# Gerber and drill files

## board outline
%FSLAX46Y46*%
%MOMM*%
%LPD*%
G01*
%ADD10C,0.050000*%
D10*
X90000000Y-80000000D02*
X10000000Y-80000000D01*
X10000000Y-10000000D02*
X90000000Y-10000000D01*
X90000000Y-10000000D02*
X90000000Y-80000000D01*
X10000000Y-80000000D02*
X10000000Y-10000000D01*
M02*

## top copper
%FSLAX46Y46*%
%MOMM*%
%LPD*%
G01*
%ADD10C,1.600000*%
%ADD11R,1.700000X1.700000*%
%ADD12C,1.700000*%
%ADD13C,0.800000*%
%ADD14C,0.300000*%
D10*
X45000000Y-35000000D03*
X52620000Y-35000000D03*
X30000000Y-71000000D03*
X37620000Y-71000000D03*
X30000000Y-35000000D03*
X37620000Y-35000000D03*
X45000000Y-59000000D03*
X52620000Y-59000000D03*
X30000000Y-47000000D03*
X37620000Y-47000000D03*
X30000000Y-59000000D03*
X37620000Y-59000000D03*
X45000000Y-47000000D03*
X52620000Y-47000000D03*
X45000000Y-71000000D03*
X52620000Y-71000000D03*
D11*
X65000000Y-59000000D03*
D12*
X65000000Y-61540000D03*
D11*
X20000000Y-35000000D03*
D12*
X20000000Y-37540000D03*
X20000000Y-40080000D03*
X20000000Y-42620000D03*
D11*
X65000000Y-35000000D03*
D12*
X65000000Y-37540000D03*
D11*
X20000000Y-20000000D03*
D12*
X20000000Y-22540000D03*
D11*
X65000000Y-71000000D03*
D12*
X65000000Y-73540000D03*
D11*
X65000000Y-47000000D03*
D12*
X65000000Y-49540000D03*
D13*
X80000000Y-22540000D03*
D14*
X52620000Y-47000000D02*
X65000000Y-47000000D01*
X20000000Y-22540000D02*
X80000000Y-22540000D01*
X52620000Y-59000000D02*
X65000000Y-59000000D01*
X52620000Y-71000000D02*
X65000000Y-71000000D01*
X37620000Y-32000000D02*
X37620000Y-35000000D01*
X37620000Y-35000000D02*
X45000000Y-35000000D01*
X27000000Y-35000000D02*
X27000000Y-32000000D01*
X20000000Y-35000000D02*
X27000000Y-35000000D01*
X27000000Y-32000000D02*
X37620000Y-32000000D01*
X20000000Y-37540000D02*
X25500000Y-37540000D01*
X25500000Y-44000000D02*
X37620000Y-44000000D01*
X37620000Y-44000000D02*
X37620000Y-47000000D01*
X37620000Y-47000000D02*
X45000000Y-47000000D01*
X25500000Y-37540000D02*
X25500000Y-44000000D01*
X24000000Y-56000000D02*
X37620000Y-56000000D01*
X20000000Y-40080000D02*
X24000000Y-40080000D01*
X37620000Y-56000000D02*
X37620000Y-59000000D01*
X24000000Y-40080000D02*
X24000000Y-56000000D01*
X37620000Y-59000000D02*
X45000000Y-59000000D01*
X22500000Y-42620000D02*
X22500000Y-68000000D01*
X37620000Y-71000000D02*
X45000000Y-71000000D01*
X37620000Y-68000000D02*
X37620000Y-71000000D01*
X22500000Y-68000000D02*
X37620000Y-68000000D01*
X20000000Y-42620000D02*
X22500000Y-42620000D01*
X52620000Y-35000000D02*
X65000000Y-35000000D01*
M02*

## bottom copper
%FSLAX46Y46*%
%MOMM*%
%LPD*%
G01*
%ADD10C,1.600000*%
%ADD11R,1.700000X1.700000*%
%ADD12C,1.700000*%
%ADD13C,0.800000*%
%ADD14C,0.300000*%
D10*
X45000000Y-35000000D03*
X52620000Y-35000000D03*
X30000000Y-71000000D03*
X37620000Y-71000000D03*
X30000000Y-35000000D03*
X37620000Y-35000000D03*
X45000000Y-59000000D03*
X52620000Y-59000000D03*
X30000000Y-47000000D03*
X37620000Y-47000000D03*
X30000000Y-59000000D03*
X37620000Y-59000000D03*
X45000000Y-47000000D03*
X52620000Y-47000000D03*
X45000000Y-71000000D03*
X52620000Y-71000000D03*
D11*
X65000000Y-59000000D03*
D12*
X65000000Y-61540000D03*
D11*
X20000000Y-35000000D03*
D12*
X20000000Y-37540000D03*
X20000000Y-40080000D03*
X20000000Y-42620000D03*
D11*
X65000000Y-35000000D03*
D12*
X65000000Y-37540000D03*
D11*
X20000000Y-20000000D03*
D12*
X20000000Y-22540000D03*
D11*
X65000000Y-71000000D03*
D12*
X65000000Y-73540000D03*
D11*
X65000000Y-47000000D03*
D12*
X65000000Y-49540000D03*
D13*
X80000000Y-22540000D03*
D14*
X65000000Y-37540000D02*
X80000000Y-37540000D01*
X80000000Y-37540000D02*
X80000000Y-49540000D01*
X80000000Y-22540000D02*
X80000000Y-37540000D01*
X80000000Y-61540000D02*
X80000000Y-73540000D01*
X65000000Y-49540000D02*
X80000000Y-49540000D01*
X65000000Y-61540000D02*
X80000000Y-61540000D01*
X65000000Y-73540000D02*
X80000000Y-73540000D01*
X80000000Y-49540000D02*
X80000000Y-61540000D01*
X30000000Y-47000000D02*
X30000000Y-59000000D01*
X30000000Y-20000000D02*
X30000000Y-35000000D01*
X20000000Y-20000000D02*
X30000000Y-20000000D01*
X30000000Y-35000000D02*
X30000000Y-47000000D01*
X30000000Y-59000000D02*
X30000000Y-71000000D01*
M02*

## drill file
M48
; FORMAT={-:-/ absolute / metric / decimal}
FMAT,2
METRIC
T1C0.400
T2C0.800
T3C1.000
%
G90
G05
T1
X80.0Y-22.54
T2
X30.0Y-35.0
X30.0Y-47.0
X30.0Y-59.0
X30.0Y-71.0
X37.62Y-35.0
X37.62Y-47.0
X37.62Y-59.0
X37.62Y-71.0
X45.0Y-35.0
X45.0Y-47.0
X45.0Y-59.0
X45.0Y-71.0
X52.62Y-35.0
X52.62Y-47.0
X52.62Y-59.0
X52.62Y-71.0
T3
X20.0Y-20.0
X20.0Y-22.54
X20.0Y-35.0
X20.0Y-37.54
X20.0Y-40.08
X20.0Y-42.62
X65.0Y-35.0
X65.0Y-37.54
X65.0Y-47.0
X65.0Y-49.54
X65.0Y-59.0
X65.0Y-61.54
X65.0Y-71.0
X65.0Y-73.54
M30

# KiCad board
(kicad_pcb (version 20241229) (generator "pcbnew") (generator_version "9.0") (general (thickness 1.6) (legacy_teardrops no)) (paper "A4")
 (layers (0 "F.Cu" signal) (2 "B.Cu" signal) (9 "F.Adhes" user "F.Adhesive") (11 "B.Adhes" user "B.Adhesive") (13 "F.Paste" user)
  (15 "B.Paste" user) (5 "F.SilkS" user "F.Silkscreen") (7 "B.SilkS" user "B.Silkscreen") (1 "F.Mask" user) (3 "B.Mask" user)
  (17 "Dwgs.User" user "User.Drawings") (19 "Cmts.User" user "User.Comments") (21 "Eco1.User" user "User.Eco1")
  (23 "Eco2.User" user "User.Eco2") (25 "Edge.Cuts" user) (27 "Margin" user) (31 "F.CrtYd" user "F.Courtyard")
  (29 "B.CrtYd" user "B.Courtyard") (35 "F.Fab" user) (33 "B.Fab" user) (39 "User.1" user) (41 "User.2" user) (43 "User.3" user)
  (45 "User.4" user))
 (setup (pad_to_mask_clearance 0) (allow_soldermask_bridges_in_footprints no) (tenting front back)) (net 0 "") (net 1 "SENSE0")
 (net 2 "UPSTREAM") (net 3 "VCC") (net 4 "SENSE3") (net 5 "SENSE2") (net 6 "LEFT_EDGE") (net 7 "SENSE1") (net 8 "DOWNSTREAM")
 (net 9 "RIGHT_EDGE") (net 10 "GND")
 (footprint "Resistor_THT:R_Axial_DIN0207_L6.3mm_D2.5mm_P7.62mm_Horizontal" (layer "F.Cu") (at 45 35)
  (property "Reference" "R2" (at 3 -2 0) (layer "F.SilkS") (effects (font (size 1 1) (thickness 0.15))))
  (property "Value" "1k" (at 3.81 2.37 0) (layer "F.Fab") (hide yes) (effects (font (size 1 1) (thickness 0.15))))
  (pad "1" thru_hole circle (at 0 0) (size 1.6 1.6) (drill 0.8) (layers "*.Cu" "*.Mask") (remove_unused_layers no) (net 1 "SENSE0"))
  (pad "2" thru_hole circle (at 7.62 0) (size 1.6 1.6) (drill 0.8) (layers "*.Cu" "*.Mask") (remove_unused_layers no) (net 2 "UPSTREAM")))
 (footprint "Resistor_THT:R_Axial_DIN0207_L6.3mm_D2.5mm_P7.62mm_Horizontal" (layer "F.Cu") (at 30 71)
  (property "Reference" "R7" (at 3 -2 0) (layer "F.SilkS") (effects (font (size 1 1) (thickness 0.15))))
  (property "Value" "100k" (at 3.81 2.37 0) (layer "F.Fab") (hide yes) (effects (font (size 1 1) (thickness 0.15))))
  (pad "1" thru_hole circle (at 0 0) (size 1.6 1.6) (drill 0.8) (layers "*.Cu" "*.Mask") (remove_unused_layers no) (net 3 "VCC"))
  (pad "2" thru_hole circle (at 7.62 0) (size 1.6 1.6) (drill 0.8) (layers "*.Cu" "*.Mask") (remove_unused_layers no) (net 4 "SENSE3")))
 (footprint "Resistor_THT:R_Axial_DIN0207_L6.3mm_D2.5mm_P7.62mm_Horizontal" (layer "F.Cu") (at 30 35)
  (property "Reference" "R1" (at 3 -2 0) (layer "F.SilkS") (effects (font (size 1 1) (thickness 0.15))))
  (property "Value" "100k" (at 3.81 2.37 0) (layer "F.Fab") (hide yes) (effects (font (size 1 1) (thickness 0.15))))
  (pad "1" thru_hole circle (at 0 0) (size 1.6 1.6) (drill 0.8) (layers "*.Cu" "*.Mask") (remove_unused_layers no) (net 3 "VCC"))
  (pad "2" thru_hole circle (at 7.62 0) (size 1.6 1.6) (drill 0.8) (layers "*.Cu" "*.Mask") (remove_unused_layers no) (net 1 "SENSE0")))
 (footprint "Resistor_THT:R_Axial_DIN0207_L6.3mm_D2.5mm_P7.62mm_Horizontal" (layer "F.Cu") (at 45 59)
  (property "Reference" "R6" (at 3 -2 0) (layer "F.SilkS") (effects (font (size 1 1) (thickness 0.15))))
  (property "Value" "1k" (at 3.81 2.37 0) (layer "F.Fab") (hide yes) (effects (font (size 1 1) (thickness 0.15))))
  (pad "1" thru_hole circle (at 0 0) (size 1.6 1.6) (drill 0.8) (layers "*.Cu" "*.Mask") (remove_unused_layers no) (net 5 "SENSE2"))
  (pad "2" thru_hole circle (at 7.62 0) (size 1.6 1.6) (drill 0.8) (layers "*.Cu" "*.Mask") (remove_unused_layers no) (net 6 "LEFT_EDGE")))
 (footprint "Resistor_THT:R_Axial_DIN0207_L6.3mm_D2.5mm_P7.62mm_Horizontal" (layer "F.Cu") (at 30 47)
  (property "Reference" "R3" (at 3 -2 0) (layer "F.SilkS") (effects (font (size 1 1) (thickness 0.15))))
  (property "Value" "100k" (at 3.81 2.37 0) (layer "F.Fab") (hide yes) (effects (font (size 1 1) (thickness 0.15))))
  (pad "1" thru_hole circle (at 0 0) (size 1.6 1.6) (drill 0.8) (layers "*.Cu" "*.Mask") (remove_unused_layers no) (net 3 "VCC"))
  (pad "2" thru_hole circle (at 7.62 0) (size 1.6 1.6) (drill 0.8) (layers "*.Cu" "*.Mask") (remove_unused_layers no) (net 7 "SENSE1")))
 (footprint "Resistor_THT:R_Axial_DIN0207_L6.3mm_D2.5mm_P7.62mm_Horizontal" (layer "F.Cu") (at 30 59)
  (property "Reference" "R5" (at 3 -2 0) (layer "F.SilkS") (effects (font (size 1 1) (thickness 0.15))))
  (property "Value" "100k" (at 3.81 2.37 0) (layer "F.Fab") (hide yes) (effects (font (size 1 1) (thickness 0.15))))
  (pad "1" thru_hole circle (at 0 0) (size 1.6 1.6) (drill 0.8) (layers "*.Cu" "*.Mask") (remove_unused_layers no) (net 3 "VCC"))
  (pad "2" thru_hole circle (at 7.62 0) (size 1.6 1.6) (drill 0.8) (layers "*.Cu" "*.Mask") (remove_unused_layers no) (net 5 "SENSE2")))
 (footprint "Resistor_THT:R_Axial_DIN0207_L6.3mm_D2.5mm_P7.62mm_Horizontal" (layer "F.Cu") (at 45 47)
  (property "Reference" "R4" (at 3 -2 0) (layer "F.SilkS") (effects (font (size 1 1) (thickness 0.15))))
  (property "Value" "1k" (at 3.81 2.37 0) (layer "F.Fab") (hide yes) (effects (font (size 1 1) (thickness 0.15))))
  (pad "1" thru_hole circle (at 0 0) (size 1.6 1.6) (drill 0.8) (layers "*.Cu" "*.Mask") (remove_unused_layers no) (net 7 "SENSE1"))
  (pad "2" thru_hole circle (at 7.62 0) (size 1.6 1.6) (drill 0.8) (layers "*.Cu" "*.Mask") (remove_unused_layers no) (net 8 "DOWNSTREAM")))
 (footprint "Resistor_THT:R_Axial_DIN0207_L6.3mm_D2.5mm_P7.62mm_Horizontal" (layer "F.Cu") (at 45 71)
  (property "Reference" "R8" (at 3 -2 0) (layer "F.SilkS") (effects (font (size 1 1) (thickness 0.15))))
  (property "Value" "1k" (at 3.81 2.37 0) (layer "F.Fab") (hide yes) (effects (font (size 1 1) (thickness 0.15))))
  (pad "1" thru_hole circle (at 0 0) (size 1.6 1.6) (drill 0.8) (layers "*.Cu" "*.Mask") (remove_unused_layers no) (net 4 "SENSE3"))
  (pad "2" thru_hole circle (at 7.62 0) (size 1.6 1.6) (drill 0.8) (layers "*.Cu" "*.Mask") (remove_unused_layers no) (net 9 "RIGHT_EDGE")))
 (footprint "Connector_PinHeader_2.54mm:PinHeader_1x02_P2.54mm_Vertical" (layer "F.Cu") (at 65 59)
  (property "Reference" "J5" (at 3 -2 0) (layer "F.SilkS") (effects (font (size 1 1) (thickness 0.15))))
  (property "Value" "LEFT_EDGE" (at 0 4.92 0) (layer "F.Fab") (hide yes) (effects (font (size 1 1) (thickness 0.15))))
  (pad "1" thru_hole rect (at 0 0) (size 1.7 1.7) (drill 1) (layers "*.Cu" "*.Mask") (remove_unused_layers no) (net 6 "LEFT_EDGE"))
  (pad "2" thru_hole circle (at 0 2.54) (size 1.7 1.7) (drill 1) (layers "*.Cu" "*.Mask") (remove_unused_layers no) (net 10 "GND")))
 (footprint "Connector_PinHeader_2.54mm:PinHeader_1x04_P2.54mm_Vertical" (layer "F.Cu") (at 20 35)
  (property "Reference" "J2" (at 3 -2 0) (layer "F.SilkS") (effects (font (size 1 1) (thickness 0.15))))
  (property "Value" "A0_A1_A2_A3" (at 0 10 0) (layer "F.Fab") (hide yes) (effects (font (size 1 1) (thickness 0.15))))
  (pad "1" thru_hole rect (at 0 0) (size 1.7 1.7) (drill 1) (layers "*.Cu" "*.Mask") (remove_unused_layers no) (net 1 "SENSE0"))
  (pad "2" thru_hole circle (at 0 2.54) (size 1.7 1.7) (drill 1) (layers "*.Cu" "*.Mask") (remove_unused_layers no) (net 7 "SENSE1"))
  (pad "3" thru_hole circle (at 0 5.08) (size 1.7 1.7) (drill 1) (layers "*.Cu" "*.Mask") (remove_unused_layers no) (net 5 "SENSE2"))
  (pad "4" thru_hole circle (at 0 7.62) (size 1.7 1.7) (drill 1) (layers "*.Cu" "*.Mask") (remove_unused_layers no) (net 4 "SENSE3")))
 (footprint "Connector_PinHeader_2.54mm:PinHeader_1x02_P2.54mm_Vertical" (layer "F.Cu") (at 65 35)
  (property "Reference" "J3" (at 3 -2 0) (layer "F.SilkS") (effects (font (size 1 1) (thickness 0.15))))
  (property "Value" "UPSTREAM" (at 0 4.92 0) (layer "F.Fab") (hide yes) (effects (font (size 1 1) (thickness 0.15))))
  (pad "1" thru_hole rect (at 0 0) (size 1.7 1.7) (drill 1) (layers "*.Cu" "*.Mask") (remove_unused_layers no) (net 2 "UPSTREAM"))
  (pad "2" thru_hole circle (at 0 2.54) (size 1.7 1.7) (drill 1) (layers "*.Cu" "*.Mask") (remove_unused_layers no) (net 10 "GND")))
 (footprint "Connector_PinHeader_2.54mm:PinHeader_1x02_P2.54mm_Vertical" (layer "F.Cu") (at 20 20)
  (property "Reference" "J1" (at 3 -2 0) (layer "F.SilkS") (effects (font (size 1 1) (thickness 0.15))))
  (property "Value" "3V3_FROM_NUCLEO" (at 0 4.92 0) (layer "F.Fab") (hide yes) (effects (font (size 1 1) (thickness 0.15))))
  (pad "1" thru_hole rect (at 0 0) (size 1.7 1.7) (drill 1) (layers "*.Cu" "*.Mask") (remove_unused_layers no) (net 3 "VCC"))
  (pad "2" thru_hole circle (at 0 2.54) (size 1.7 1.7) (drill 1) (layers "*.Cu" "*.Mask") (remove_unused_layers no) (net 10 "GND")))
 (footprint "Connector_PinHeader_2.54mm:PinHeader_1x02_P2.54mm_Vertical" (layer "F.Cu") (at 65 71)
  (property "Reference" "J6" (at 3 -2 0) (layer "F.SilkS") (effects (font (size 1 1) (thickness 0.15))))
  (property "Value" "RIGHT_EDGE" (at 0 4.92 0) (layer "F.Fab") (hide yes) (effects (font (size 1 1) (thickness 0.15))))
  (pad "1" thru_hole rect (at 0 0) (size 1.7 1.7) (drill 1) (layers "*.Cu" "*.Mask") (remove_unused_layers no) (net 9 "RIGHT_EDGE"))
  (pad "2" thru_hole circle (at 0 2.54) (size 1.7 1.7) (drill 1) (layers "*.Cu" "*.Mask") (remove_unused_layers no) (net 10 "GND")))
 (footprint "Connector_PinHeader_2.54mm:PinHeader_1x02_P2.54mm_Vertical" (layer "F.Cu") (at 65 47)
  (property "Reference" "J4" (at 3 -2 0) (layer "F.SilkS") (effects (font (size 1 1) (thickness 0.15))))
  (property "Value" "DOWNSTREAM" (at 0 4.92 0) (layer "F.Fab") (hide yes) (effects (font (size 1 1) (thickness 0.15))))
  (pad "1" thru_hole rect (at 0 0) (size 1.7 1.7) (drill 1) (layers "*.Cu" "*.Mask") (remove_unused_layers no) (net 8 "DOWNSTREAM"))
  (pad "2" thru_hole circle (at 0 2.54) (size 1.7 1.7) (drill 1) (layers "*.Cu" "*.Mask") (remove_unused_layers no) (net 10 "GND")))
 (gr_line (start 90 80) (end 10 80) (stroke (width 0.05) (type default)) (layer "Edge.Cuts"))
 (gr_line (start 10 10) (end 90 10) (stroke (width 0.05) (type default)) (layer "Edge.Cuts"))
 (gr_line (start 90 10) (end 90 80) (stroke (width 0.05) (type default)) (layer "Edge.Cuts"))
 (gr_line (start 10 80) (end 10 10) (stroke (width 0.05) (type default)) (layer "Edge.Cuts"))
 (segment (start 52.62 47) (end 65 47) (width 0.3) (layer "F.Cu") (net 8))
 (segment (start 20 22.54) (end 80 22.54) (width 0.3) (layer "F.Cu") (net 10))
 (via (at 80 22.54) (size 0.8) (drill 0.4) (layers "F.Cu" "B.Cu") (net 10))
 (segment (start 65 37.54) (end 80 37.54) (width 0.3) (layer "B.Cu") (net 10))
 (segment (start 80 37.54) (end 80 49.54) (width 0.3) (layer "B.Cu") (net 10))
 (segment (start 80 22.54) (end 80 37.54) (width 0.3) (layer "B.Cu") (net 10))
 (segment (start 80 61.54) (end 80 73.54) (width 0.3) (layer "B.Cu") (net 10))
 (segment (start 65 49.54) (end 80 49.54) (width 0.3) (layer "B.Cu") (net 10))
 (segment (start 65 61.54) (end 80 61.54) (width 0.3) (layer "B.Cu") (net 10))
 (segment (start 65 73.54) (end 80 73.54) (width 0.3) (layer "B.Cu") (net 10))
 (segment (start 80 49.54) (end 80 61.54) (width 0.3) (layer "B.Cu") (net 10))
 (segment (start 52.62 59) (end 65 59) (width 0.3) (layer "F.Cu") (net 6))
 (segment (start 52.62 71) (end 65 71) (width 0.3) (layer "F.Cu") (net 9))
 (segment (start 37.62 32) (end 37.62 35) (width 0.3) (layer "F.Cu") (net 1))
 (segment (start 37.62 35) (end 45 35) (width 0.3) (layer "F.Cu") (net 1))
 (segment (start 27 35) (end 27 32) (width 0.3) (layer "F.Cu") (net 1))
 (segment (start 20 35) (end 27 35) (width 0.3) (layer "F.Cu") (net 1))
 (segment (start 27 32) (end 37.62 32) (width 0.3) (layer "F.Cu") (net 1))
 (segment (start 20 37.54) (end 25.5 37.54) (width 0.3) (layer "F.Cu") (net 7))
 (segment (start 25.5 44) (end 37.62 44) (width 0.3) (layer "F.Cu") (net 7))
 (segment (start 37.62 44) (end 37.62 47) (width 0.3) (layer "F.Cu") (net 7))
 (segment (start 37.62 47) (end 45 47) (width 0.3) (layer "F.Cu") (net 7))
 (segment (start 25.5 37.54) (end 25.5 44) (width 0.3) (layer "F.Cu") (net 7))
 (segment (start 24 56) (end 37.62 56) (width 0.3) (layer "F.Cu") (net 5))
 (segment (start 20 40.08) (end 24 40.08) (width 0.3) (layer "F.Cu") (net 5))
 (segment (start 37.62 56) (end 37.62 59) (width 0.3) (layer "F.Cu") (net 5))
 (segment (start 24 40.08) (end 24 56) (width 0.3) (layer "F.Cu") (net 5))
 (segment (start 37.62 59) (end 45 59) (width 0.3) (layer "F.Cu") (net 5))
 (segment (start 22.5 42.62) (end 22.5 68) (width 0.3) (layer "F.Cu") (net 4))
 (segment (start 37.62 71) (end 45 71) (width 0.3) (layer "F.Cu") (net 4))
 (segment (start 37.62 68) (end 37.62 71) (width 0.3) (layer "F.Cu") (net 4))
 (segment (start 22.5 68) (end 37.62 68) (width 0.3) (layer "F.Cu") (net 4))
 (segment (start 20 42.62) (end 22.5 42.62) (width 0.3) (layer "F.Cu") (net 4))
 (segment (start 52.62 35) (end 65 35) (width 0.3) (layer "F.Cu") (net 2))
 (segment (start 30 47) (end 30 59) (width 0.3) (layer "B.Cu") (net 3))
 (segment (start 30 20) (end 30 35) (width 0.3) (layer "B.Cu") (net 3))
 (segment (start 20 20) (end 30 20) (width 0.3) (layer "B.Cu") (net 3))
 (segment (start 30 35) (end 30 47) (width 0.3) (layer "B.Cu") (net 3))
 (segment (start 30 59) (end 30 71) (width 0.3) (layer "B.Cu") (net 3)))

